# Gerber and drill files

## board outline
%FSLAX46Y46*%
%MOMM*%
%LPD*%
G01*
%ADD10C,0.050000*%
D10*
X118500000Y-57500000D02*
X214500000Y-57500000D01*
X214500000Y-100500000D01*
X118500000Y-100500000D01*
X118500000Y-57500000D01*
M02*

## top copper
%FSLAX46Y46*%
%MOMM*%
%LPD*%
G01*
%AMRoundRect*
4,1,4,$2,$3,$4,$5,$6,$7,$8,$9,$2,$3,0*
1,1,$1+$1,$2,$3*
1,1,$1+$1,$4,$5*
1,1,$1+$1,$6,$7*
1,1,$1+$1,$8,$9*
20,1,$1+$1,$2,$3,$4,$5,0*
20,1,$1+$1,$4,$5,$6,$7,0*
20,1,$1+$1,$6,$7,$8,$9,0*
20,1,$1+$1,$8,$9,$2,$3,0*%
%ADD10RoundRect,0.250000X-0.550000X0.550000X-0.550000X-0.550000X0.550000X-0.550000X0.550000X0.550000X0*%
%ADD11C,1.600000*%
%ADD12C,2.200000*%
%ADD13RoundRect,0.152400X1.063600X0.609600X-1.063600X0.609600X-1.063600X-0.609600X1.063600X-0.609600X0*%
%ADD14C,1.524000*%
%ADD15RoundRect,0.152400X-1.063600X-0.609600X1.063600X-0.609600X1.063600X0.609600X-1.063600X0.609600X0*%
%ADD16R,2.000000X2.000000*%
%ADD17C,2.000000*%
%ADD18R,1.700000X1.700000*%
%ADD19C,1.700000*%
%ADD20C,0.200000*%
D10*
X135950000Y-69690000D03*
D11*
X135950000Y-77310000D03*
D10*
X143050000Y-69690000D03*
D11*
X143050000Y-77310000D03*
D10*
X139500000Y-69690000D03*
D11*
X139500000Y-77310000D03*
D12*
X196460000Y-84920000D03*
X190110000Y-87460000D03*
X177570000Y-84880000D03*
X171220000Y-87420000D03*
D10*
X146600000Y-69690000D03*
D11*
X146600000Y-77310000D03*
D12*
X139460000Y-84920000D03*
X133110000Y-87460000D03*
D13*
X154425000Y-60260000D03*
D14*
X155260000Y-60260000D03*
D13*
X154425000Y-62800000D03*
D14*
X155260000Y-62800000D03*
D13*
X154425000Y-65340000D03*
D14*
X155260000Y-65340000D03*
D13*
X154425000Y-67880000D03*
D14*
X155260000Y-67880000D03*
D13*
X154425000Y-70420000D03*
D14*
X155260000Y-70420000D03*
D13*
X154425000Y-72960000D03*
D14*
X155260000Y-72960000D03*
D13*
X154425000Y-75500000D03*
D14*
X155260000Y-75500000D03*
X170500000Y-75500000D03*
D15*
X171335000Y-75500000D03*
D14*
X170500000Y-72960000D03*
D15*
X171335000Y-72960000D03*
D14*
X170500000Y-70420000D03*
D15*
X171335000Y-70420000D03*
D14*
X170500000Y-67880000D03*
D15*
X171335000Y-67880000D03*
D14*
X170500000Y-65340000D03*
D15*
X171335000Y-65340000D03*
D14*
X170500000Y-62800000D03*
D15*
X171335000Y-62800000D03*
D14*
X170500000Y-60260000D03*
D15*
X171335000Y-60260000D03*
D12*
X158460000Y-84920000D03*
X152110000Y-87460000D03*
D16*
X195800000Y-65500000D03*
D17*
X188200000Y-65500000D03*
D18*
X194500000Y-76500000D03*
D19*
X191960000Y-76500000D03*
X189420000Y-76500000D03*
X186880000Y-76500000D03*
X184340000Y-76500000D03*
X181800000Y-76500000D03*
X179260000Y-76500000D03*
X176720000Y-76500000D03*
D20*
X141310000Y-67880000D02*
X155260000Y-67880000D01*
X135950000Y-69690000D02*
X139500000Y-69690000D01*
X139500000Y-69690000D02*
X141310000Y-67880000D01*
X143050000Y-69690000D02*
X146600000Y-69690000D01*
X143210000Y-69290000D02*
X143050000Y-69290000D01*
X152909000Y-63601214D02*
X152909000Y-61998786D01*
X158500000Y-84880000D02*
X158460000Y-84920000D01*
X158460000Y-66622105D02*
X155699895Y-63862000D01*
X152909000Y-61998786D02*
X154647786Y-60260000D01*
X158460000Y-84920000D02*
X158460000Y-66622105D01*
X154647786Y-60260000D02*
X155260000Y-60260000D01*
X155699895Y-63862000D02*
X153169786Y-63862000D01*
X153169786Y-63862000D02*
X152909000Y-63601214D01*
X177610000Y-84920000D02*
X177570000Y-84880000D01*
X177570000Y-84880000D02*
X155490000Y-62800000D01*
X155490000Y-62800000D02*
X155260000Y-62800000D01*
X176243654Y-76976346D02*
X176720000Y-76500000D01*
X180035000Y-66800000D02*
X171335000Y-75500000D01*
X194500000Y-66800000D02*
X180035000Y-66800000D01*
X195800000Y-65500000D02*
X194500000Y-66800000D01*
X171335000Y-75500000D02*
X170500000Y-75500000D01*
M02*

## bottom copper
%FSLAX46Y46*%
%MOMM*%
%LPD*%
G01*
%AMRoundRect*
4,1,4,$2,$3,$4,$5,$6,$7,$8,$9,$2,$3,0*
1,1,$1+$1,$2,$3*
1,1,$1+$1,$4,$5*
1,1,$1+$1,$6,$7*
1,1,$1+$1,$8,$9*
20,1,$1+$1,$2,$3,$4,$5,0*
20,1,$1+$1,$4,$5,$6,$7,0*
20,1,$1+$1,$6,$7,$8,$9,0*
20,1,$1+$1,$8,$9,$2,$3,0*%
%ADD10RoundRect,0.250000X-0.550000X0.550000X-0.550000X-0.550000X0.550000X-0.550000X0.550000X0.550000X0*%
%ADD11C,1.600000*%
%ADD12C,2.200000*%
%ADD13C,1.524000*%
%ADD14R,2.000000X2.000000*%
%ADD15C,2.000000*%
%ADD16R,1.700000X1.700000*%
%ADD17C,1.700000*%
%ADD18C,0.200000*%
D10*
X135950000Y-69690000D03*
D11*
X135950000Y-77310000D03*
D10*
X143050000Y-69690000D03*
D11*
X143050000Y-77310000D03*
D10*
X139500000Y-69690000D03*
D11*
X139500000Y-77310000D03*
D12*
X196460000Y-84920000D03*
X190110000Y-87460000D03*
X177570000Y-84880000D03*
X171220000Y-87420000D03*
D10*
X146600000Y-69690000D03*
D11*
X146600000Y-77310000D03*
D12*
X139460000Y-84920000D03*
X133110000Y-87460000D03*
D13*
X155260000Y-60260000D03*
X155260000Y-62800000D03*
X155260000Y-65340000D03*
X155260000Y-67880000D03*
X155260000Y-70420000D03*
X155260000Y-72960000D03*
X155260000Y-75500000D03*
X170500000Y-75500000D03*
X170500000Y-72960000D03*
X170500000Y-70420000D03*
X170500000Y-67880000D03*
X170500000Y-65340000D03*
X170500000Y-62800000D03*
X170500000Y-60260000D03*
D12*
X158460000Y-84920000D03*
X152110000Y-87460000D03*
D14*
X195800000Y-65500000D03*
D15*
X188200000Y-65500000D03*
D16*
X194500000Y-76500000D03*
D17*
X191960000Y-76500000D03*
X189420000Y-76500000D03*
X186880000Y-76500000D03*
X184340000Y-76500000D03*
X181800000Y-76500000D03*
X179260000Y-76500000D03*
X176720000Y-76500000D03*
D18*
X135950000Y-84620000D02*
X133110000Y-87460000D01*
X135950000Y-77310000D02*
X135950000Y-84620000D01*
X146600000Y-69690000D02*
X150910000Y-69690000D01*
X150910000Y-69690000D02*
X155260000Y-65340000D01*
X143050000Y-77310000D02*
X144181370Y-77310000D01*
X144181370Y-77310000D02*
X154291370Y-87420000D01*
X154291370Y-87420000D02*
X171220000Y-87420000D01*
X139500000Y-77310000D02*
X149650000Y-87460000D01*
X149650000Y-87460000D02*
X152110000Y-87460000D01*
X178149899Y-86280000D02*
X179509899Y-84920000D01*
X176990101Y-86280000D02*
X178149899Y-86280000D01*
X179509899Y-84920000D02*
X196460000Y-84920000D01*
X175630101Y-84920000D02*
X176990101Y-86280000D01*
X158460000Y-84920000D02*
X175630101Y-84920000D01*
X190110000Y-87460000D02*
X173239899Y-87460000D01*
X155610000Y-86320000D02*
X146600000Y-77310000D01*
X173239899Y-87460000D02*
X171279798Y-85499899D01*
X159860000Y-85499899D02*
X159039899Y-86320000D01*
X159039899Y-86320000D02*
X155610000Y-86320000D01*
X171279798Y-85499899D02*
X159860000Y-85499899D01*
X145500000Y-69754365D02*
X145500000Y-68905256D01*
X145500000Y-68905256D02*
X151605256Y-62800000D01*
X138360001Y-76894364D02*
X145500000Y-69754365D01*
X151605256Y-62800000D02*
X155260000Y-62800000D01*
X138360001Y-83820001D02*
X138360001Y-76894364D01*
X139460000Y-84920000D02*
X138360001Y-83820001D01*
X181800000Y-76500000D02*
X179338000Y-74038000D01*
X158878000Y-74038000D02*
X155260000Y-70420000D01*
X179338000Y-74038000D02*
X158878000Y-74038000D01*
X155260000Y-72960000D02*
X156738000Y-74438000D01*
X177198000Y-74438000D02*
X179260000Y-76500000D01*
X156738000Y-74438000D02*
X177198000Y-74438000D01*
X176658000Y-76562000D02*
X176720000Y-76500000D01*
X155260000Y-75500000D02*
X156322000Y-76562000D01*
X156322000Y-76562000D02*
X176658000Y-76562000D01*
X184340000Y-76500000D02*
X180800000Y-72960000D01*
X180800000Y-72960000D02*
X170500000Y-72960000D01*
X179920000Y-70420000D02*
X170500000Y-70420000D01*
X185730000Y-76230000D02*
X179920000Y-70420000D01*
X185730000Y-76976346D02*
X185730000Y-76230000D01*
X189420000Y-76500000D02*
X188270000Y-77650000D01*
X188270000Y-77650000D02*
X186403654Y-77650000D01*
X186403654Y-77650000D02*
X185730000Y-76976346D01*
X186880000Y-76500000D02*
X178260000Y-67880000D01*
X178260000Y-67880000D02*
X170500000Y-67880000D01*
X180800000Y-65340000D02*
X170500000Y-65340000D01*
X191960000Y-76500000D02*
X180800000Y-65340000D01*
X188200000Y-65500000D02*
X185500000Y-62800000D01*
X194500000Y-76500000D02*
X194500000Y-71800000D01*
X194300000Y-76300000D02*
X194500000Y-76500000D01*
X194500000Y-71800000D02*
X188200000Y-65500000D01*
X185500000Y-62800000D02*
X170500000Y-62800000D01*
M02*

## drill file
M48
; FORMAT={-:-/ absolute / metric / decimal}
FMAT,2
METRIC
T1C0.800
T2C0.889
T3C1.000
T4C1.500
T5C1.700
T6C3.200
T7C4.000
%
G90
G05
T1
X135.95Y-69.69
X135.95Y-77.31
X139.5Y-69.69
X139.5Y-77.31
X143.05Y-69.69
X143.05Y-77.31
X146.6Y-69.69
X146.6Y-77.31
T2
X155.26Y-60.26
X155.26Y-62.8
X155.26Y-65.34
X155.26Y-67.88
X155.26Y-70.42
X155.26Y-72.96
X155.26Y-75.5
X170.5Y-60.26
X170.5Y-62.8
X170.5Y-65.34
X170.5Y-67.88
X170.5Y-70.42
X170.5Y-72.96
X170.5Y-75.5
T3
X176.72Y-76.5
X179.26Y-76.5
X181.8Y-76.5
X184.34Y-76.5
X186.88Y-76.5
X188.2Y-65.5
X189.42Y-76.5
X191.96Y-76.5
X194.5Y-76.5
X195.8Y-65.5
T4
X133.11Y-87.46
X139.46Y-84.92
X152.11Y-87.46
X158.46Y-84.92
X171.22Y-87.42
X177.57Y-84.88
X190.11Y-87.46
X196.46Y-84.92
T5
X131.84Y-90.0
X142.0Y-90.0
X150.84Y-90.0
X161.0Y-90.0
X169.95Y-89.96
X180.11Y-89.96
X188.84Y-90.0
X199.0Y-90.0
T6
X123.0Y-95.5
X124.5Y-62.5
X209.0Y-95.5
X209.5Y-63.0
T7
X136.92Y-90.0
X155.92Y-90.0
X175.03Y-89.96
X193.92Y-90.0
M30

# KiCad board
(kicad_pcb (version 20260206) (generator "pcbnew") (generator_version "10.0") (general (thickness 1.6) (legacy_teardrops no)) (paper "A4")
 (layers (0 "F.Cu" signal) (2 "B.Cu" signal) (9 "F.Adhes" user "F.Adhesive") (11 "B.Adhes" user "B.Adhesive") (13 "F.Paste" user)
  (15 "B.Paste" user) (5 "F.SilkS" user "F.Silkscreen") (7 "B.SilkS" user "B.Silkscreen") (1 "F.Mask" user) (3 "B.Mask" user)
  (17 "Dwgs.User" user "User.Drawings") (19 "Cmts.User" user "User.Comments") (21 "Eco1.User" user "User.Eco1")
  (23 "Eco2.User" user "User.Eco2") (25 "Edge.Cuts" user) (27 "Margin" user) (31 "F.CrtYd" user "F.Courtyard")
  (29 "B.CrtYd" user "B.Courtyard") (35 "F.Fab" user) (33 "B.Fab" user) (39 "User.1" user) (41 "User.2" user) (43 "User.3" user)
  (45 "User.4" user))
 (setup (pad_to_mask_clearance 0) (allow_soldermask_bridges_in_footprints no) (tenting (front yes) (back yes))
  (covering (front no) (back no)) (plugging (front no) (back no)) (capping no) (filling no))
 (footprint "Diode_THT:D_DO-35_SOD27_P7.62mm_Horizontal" (layer "F.Cu") (at 135.95 69.69 -90)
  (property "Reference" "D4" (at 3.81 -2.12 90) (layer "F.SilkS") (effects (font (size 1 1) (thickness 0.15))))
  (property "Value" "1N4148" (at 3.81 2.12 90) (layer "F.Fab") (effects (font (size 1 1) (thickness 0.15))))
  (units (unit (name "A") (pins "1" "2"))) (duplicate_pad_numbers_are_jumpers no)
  (pad "1" thru_hole roundrect (at 0 0 270) (size 1.6 1.6) (drill 0.8) (layers "*.Cu" "*.Mask") (remove_unused_layers no)
   (roundrect_rratio 0.15625) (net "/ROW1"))
  (pad "2" thru_hole circle (at 7.62 0 270) (size 1.6 1.6) (drill 0.8) (layers "*.Cu" "*.Mask") (remove_unused_layers no) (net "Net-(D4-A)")))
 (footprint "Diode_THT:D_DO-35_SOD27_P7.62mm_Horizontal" (layer "F.Cu") (at 143.05 69.69 -90)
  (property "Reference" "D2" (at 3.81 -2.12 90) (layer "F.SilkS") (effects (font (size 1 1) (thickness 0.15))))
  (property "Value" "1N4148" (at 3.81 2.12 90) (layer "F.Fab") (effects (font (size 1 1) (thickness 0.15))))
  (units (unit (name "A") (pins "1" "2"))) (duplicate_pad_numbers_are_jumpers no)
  (pad "1" thru_hole roundrect (at 0 0 270) (size 1.6 1.6) (drill 0.8) (layers "*.Cu" "*.Mask") (remove_unused_layers no)
   (roundrect_rratio 0.15625) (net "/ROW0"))
  (pad "2" thru_hole circle (at 7.62 0 270) (size 1.6 1.6) (drill 0.8) (layers "*.Cu" "*.Mask") (remove_unused_layers no) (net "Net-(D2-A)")))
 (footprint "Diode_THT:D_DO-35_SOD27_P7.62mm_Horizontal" (layer "F.Cu") (at 139.5 69.69 -90)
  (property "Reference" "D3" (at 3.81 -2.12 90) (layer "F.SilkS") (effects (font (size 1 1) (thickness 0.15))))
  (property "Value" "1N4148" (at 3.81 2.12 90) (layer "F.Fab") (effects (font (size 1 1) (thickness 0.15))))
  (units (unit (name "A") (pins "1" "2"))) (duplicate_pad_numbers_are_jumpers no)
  (pad "1" thru_hole roundrect (at 0 0 270) (size 1.6 1.6) (drill 0.8) (layers "*.Cu" "*.Mask") (remove_unused_layers no)
   (roundrect_rratio 0.15625) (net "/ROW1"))
  (pad "2" thru_hole circle (at 7.62 0 270) (size 1.6 1.6) (drill 0.8) (layers "*.Cu" "*.Mask") (remove_unused_layers no) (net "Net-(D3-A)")))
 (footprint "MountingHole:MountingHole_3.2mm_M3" (layer "F.Cu") (at 124.5 62.5)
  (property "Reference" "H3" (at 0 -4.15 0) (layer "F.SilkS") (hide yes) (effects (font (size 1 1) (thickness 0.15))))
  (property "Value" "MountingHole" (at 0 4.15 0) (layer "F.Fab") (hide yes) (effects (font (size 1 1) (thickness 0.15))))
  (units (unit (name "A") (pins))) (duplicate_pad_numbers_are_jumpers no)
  (pad "" np_thru_hole circle (at 0 0) (size 3.2 3.2) (drill 3.2) (layers "*.Cu" "*.Mask")))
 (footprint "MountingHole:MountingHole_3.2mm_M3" (layer "F.Cu") (at 209 95.5)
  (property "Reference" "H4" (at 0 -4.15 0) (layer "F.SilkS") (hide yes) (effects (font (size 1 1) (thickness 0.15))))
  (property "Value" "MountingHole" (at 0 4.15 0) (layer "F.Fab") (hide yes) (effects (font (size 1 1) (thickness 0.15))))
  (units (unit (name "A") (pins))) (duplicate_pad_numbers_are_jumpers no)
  (pad "" np_thru_hole circle (at 0 0) (size 3.2 3.2) (drill 3.2) (layers "*.Cu" "*.Mask")))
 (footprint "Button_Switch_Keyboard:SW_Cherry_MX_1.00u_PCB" (layer "F.Cu") (at 196.46 84.92)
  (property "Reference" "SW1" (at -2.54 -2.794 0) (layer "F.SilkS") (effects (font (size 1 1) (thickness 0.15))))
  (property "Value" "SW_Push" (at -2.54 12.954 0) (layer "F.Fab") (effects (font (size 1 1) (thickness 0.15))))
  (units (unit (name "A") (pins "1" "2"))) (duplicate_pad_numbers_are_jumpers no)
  (pad "" np_thru_hole circle (at -7.62 5.08) (size 1.7 1.7) (drill 1.7) (layers "*.Cu" "*.Mask"))
  (pad "" np_thru_hole circle (at -2.54 5.08) (size 4 4) (drill 4) (layers "*.Cu" "*.Mask"))
  (pad "" np_thru_hole circle (at 2.54 5.08) (size 1.7 1.7) (drill 1.7) (layers "*.Cu" "*.Mask"))
  (pad "1" thru_hole circle (at 0 0) (size 2.2 2.2) (drill 1.5) (layers "*.Cu" "*.Mask") (remove_unused_layers no) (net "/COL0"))
  (pad "2" thru_hole circle (at -6.35 2.54) (size 2.2 2.2) (drill 1.5) (layers "*.Cu" "*.Mask") (remove_unused_layers no) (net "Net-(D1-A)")))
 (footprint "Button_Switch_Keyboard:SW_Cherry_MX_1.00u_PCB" (layer "F.Cu") (at 177.57 84.88)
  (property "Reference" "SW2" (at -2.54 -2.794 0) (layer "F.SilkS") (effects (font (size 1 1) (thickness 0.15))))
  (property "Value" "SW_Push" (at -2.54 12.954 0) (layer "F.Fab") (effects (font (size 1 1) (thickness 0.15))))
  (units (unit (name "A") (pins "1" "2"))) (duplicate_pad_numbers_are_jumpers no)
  (pad "" np_thru_hole circle (at -7.62 5.08) (size 1.7 1.7) (drill 1.7) (layers "*.Cu" "*.Mask"))
  (pad "" np_thru_hole circle (at -2.54 5.08) (size 4 4) (drill 4) (layers "*.Cu" "*.Mask"))
  (pad "" np_thru_hole circle (at 2.54 5.08) (size 1.7 1.7) (drill 1.7) (layers "*.Cu" "*.Mask"))
  (pad "1" thru_hole circle (at 0 0) (size 2.2 2.2) (drill 1.5) (layers "*.Cu" "*.Mask") (remove_unused_layers no) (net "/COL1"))
  (pad "2" thru_hole circle (at -6.35 2.54) (size 2.2 2.2) (drill 1.5) (layers "*.Cu" "*.Mask") (remove_unused_layers no) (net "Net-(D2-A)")))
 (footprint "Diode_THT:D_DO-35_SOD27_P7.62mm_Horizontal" (layer "F.Cu") (at 146.6 69.69 -90)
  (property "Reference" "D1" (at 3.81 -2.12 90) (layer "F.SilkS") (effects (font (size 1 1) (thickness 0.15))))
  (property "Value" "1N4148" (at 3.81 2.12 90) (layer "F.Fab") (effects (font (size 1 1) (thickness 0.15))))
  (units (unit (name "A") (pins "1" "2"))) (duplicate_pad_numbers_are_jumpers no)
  (pad "1" thru_hole roundrect (at 0 0 270) (size 1.6 1.6) (drill 0.8) (layers "*.Cu" "*.Mask") (remove_unused_layers no)
   (roundrect_rratio 0.15625) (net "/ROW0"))
  (pad "2" thru_hole circle (at 7.62 0 270) (size 1.6 1.6) (drill 0.8) (layers "*.Cu" "*.Mask") (remove_unused_layers no) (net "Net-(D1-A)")))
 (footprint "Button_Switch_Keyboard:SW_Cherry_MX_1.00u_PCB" (layer "F.Cu") (at 139.46 84.92)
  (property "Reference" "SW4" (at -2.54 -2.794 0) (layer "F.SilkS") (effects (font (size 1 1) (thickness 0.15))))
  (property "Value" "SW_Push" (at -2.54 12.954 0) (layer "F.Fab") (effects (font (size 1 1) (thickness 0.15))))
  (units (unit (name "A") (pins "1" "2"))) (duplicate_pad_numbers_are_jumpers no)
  (pad "" np_thru_hole circle (at -7.62 5.08) (size 1.7 1.7) (drill 1.7) (layers "*.Cu" "*.Mask"))
  (pad "" np_thru_hole circle (at -2.54 5.08) (size 4 4) (drill 4) (layers "*.Cu" "*.Mask"))
  (pad "" np_thru_hole circle (at 2.54 5.08) (size 1.7 1.7) (drill 1.7) (layers "*.Cu" "*.Mask"))
  (pad "1" thru_hole circle (at 0 0) (size 2.2 2.2) (drill 1.5) (layers "*.Cu" "*.Mask") (remove_unused_layers no) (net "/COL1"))
  (pad "2" thru_hole circle (at -6.35 2.54) (size 2.2 2.2) (drill 1.5) (layers "*.Cu" "*.Mask") (remove_unused_layers no) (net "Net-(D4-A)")))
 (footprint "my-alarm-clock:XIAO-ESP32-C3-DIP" (layer "F.Cu") (at 162.88 67.88 90)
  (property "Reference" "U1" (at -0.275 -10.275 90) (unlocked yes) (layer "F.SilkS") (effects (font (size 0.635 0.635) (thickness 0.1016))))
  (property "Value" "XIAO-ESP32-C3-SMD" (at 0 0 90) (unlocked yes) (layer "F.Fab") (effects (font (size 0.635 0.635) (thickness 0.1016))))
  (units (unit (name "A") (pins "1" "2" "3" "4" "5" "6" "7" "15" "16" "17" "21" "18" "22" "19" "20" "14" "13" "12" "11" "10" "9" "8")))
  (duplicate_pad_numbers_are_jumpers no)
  (pad "1" smd roundrect (at 7.62 -8.455 180) (size 2.432 1.524) (layers "F.Cu" "F.Mask") (roundrect_rratio 0.1) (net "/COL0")
   (thermal_bridge_angle 45))
  (pad "1" thru_hole circle (at 7.62 -7.62 180) (size 1.524 1.524) (drill 0.889) (layers "*.Cu" "*.Mask") (remove_unused_layers no)
   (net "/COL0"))
  (pad "2" smd roundrect (at 5.08 -8.455 180) (size 2.432 1.524) (layers "F.Cu" "F.Mask") (roundrect_rratio 0.1) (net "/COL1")
   (thermal_bridge_angle 45))
  (pad "2" thru_hole circle (at 5.08 -7.62 180) (size 1.524 1.524) (drill 0.889) (layers "*.Cu" "*.Mask") (remove_unused_layers no)
   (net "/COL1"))
  (pad "3" smd roundrect (at 2.54 -8.455 180) (size 2.432 1.524) (layers "F.Cu" "F.Mask") (roundrect_rratio 0.1) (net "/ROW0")
   (thermal_bridge_angle 45))
  (pad "3" thru_hole circle (at 2.54 -7.62 180) (size 1.524 1.524) (drill 0.889) (layers "*.Cu" "*.Mask") (remove_unused_layers no)
   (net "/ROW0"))
  (pad "4" smd roundrect (at 0 -8.455 180) (size 2.432 1.524) (layers "F.Cu" "F.Mask") (roundrect_rratio 0.1) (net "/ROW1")
   (thermal_bridge_angle 45))
  (pad "4" thru_hole circle (at 0 -7.62 180) (size 1.524 1.524) (drill 0.889) (layers "*.Cu" "*.Mask") (remove_unused_layers no)
   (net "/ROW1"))
  (pad "5" smd roundrect (at -2.54 -8.455 180) (size 2.432 1.524) (layers "F.Cu" "F.Mask") (roundrect_rratio 0.1) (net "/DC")
   (thermal_bridge_angle 45))
  (pad "5" thru_hole circle (at -2.54 -7.62 180) (size 1.524 1.524) (drill 0.889) (layers "*.Cu" "*.Mask") (remove_unused_layers no)
   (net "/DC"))
  (pad "6" smd roundrect (at -5.08 -8.455 180) (size 2.432 1.524) (layers "F.Cu" "F.Mask") (roundrect_rratio 0.1) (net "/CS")
   (thermal_bridge_angle 45))
  (pad "6" thru_hole circle (at -5.08 -7.62 180) (size 1.524 1.524) (drill 0.889) (layers "*.Cu" "*.Mask") (remove_unused_layers no)
   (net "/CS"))
  (pad "7" smd roundrect (at -7.62 -8.455 180) (size 2.432 1.524) (layers "F.Cu" "F.Mask") (roundrect_rratio 0.1) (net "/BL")
   (thermal_bridge_angle 45))
  (pad "7" thru_hole circle (at -7.62 -7.62 180) (size 1.524 1.524) (drill 0.889) (layers "*.Cu" "*.Mask") (remove_unused_layers no)
   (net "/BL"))
  (pad "8" thru_hole circle (at -7.62 7.62) (size 1.524 1.524) (drill 0.889) (layers "*.Cu" "*.Mask") (remove_unused_layers no)
   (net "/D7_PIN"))
  (pad "8" smd roundrect (at -7.62 8.455) (size 2.432 1.524) (layers "F.Cu" "F.Mask") (roundrect_rratio 0.1) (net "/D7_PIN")
   (thermal_bridge_angle 45))
  (pad "9" thru_hole circle (at -5.08 7.62) (size 1.524 1.524) (drill 0.889) (layers "*.Cu" "*.Mask") (remove_unused_layers no) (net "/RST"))
  (pad "9" smd roundrect (at -5.08 8.455) (size 2.432 1.524) (layers "F.Cu" "F.Mask") (roundrect_rratio 0.1) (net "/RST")
   (thermal_bridge_angle 45))
  (pad "10" thru_hole circle (at -2.54 7.62) (size 1.524 1.524) (drill 0.889) (layers "*.Cu" "*.Mask") (remove_unused_layers no)
   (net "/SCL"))
  (pad "10" smd roundrect (at -2.54 8.455) (size 2.432 1.524) (layers "F.Cu" "F.Mask") (roundrect_rratio 0.1) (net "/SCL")
   (thermal_bridge_angle 45))
  (pad "11" thru_hole circle (at 0 7.62) (size 1.524 1.524) (drill 0.889) (layers "*.Cu" "*.Mask") (remove_unused_layers no) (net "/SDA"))
  (pad "11" smd roundrect (at 0 8.455) (size 2.432 1.524) (layers "F.Cu" "F.Mask") (roundrect_rratio 0.1) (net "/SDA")
   (thermal_bridge_angle 45))
  (pad "12" thru_hole circle (at 2.54 7.62) (size 1.524 1.524) (drill 0.889) (layers "*.Cu" "*.Mask") (remove_unused_layers no)
   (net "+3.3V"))
  (pad "12" smd roundrect (at 2.54 8.455) (size 2.432 1.524) (layers "F.Cu" "F.Mask") (roundrect_rratio 0.1) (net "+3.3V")
   (thermal_bridge_angle 45))
  (pad "13" thru_hole circle (at 5.08 7.62) (size 1.524 1.524) (drill 0.889) (layers "*.Cu" "*.Mask") (remove_unused_layers no) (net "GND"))
  (pad "13" smd roundrect (at 5.08 8.455) (size 2.432 1.524) (layers "F.Cu" "F.Mask") (roundrect_rratio 0.1) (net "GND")
   (thermal_bridge_angle 45))
  (pad "14" thru_hole circle (at 7.62 7.62) (size 1.524 1.524) (drill 0.889) (layers "*.Cu" "*.Mask") (remove_unused_layers no)
   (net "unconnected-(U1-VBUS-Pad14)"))
  (pad "14" smd roundrect (at 7.62 8.455) (size 2.432 1.524) (layers "F.Cu" "F.Mask") (roundrect_rratio 0.1)
   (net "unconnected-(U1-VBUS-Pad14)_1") (thermal_bridge_angle 45)))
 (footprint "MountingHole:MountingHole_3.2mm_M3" (layer "F.Cu") (at 209.5 63)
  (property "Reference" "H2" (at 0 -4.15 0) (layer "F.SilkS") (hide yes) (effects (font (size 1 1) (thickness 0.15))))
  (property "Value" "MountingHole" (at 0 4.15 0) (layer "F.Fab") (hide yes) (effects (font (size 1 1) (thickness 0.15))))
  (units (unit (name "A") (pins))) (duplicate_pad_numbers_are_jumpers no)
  (pad "" np_thru_hole circle (at 0 0) (size 3.2 3.2) (drill 3.2) (layers "*.Cu" "*.Mask")))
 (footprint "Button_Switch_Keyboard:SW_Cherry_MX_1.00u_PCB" (layer "F.Cu") (at 158.46 84.92)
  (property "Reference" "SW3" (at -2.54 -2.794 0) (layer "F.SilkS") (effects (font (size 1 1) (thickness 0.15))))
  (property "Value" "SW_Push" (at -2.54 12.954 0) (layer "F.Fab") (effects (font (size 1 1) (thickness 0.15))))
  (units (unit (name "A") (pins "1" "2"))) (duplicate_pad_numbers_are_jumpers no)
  (pad "" np_thru_hole circle (at -7.62 5.08) (size 1.7 1.7) (drill 1.7) (layers "*.Cu" "*.Mask"))
  (pad "" np_thru_hole circle (at -2.54 5.08) (size 4 4) (drill 4) (layers "*.Cu" "*.Mask"))
  (pad "" np_thru_hole circle (at 2.54 5.08) (size 1.7 1.7) (drill 1.7) (layers "*.Cu" "*.Mask"))
  (pad "1" thru_hole circle (at 0 0) (size 2.2 2.2) (drill 1.5) (layers "*.Cu" "*.Mask") (remove_unused_layers no) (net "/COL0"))
  (pad "2" thru_hole circle (at -6.35 2.54) (size 2.2 2.2) (drill 1.5) (layers "*.Cu" "*.Mask") (remove_unused_layers no) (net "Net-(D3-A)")))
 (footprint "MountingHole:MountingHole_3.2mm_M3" (layer "F.Cu") (at 123 95.5)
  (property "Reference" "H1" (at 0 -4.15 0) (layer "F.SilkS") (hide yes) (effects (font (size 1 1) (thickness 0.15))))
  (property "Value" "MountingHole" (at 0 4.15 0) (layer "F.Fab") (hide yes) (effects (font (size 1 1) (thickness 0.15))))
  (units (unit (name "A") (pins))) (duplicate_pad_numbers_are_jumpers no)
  (pad "" np_thru_hole circle (at 0 0) (size 3.2 3.2) (drill 3.2) (layers "*.Cu" "*.Mask")))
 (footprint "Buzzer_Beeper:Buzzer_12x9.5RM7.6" (layer "B.Cu") (at 195.8 65.5 180)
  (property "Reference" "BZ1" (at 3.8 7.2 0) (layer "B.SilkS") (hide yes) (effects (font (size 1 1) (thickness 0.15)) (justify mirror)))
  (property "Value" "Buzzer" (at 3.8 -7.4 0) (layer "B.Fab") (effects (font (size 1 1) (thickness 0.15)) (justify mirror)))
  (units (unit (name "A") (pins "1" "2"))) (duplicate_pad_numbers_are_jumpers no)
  (pad "1" thru_hole rect (at 0 0 180) (size 2 2) (drill 1) (layers "*.Cu" "*.Mask") (remove_unused_layers no) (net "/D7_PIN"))
  (pad "2" thru_hole circle (at 7.6 0 180) (size 2 2) (drill 1) (layers "*.Cu" "*.Mask") (remove_unused_layers no) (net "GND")))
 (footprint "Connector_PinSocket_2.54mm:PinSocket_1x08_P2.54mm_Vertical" (layer "B.Cu") (at 194.5 76.5 90)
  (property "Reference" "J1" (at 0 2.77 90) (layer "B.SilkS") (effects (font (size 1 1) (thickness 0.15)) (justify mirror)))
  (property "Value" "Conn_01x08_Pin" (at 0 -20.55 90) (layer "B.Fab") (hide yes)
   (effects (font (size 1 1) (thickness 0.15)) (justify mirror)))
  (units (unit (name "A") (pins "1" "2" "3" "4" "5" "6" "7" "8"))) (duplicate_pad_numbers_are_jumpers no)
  (pad "1" thru_hole rect (at 0 0 90) (size 1.7 1.7) (drill 1) (layers "*.Cu" "*.Mask") (remove_unused_layers no) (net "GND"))
  (pad "2" thru_hole circle (at 0 -2.54 90) (size 1.7 1.7) (drill 1) (layers "*.Cu" "*.Mask") (remove_unused_layers no) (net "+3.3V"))
  (pad "3" thru_hole circle (at 0 -5.08 90) (size 1.7 1.7) (drill 1) (layers "*.Cu" "*.Mask") (remove_unused_layers no) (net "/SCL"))
  (pad "4" thru_hole circle (at 0 -7.62 90) (size 1.7 1.7) (drill 1) (layers "*.Cu" "*.Mask") (remove_unused_layers no) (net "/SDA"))
  (pad "5" thru_hole circle (at 0 -10.16 90) (size 1.7 1.7) (drill 1) (layers "*.Cu" "*.Mask") (remove_unused_layers no) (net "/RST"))
  (pad "6" thru_hole circle (at 0 -12.7 90) (size 1.7 1.7) (drill 1) (layers "*.Cu" "*.Mask") (remove_unused_layers no) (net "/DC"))
  (pad "7" thru_hole circle (at 0 -15.24 90) (size 1.7 1.7) (drill 1) (layers "*.Cu" "*.Mask") (remove_unused_layers no) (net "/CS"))
  (pad "8" thru_hole circle (at 0 -17.78 90) (size 1.7 1.7) (drill 1) (layers "*.Cu" "*.Mask") (remove_unused_layers no) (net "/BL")))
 (gr_rect (start 118.5 57.5) (end 214.5 100.5) (stroke (width 0.05) (type default)) (fill no) (layer "Edge.Cuts"))
 (segment (start 141.31 67.88) (end 155.26 67.88) (width 0.2) (layer "F.Cu") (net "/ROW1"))
 (segment (start 135.95 69.69) (end 139.5 69.69) (width 0.2) (layer "F.Cu") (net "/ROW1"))
 (segment (start 139.5 69.69) (end 141.31 67.88) (width 0.2) (layer "F.Cu") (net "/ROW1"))
 (segment (start 135.95 84.62) (end 133.11 87.46) (width 0.2) (layer "B.Cu") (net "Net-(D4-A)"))
 (segment (start 135.95 77.31) (end 135.95 84.62) (width 0.2) (layer "B.Cu") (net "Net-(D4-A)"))
 (segment (start 143.05 69.69) (end 146.6 69.69) (width 0.2) (layer "F.Cu") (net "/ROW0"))
 (segment (start 143.21 69.29) (end 143.05 69.29) (width 0.2) (layer "F.Cu") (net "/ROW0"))
 (segment (start 146.6 69.69) (end 150.91 69.69) (width 0.2) (layer "B.Cu") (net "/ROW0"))
 (segment (start 150.91 69.69) (end 155.26 65.34) (width 0.2) (layer "B.Cu") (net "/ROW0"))
 (segment (start 143.05 77.31) (end 144.18137 77.31) (width 0.2) (layer "B.Cu") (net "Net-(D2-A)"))
 (segment (start 144.18137 77.31) (end 154.29137 87.42) (width 0.2) (layer "B.Cu") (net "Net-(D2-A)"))
 (segment (start 154.29137 87.42) (end 171.22 87.42) (width 0.2) (layer "B.Cu") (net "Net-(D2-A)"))
 (segment (start 139.5 77.31) (end 149.65 87.46) (width 0.2) (layer "B.Cu") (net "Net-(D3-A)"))
 (segment (start 149.65 87.46) (end 152.11 87.46) (width 0.2) (layer "B.Cu") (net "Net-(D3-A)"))
 (segment (start 152.909 63.601214) (end 152.909 61.998786) (width 0.2) (layer "F.Cu") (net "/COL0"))
 (segment (start 158.5 84.88) (end 158.46 84.92) (width 0.2) (layer "F.Cu") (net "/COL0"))
 (segment (start 158.46 66.622105) (end 155.699895 63.862) (width 0.2) (layer "F.Cu") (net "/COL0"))
 (segment (start 152.909 61.998786) (end 154.647786 60.26) (width 0.2) (layer "F.Cu") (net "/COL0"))
 (segment (start 158.46 84.92) (end 158.46 66.622105) (width 0.2) (layer "F.Cu") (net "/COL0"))
 (segment (start 154.647786 60.26) (end 155.26 60.26) (width 0.2) (layer "F.Cu") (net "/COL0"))
 (segment (start 155.699895 63.862) (end 153.169786 63.862) (width 0.2) (layer "F.Cu") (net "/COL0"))
 (segment (start 153.169786 63.862) (end 152.909 63.601214) (width 0.2) (layer "F.Cu") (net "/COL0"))
 (segment (start 178.149899 86.28) (end 179.509899 84.92) (width 0.2) (layer "B.Cu") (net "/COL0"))
 (segment (start 176.990101 86.28) (end 178.149899 86.28) (width 0.2) (layer "B.Cu") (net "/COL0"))
 (segment (start 179.509899 84.92) (end 196.46 84.92) (width 0.2) (layer "B.Cu") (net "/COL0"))
 (segment (start 175.630101 84.92) (end 176.990101 86.28) (width 0.2) (layer "B.Cu") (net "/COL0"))
 (segment (start 158.46 84.92) (end 175.630101 84.92) (width 0.2) (layer "B.Cu") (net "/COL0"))
 (segment (start 190.11 87.46) (end 173.239899 87.46) (width 0.2) (layer "B.Cu") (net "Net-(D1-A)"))
 (segment (start 155.61 86.32) (end 146.6 77.31) (width 0.2) (layer "B.Cu") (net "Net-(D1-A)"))
 (segment (start 173.239899 87.46) (end 171.279798 85.499899) (width 0.2) (layer "B.Cu") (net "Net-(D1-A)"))
 (segment (start 159.86 85.499899) (end 159.039899 86.32) (width 0.2) (layer "B.Cu") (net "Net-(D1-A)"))
 (segment (start 159.039899 86.32) (end 155.61 86.32) (width 0.2) (layer "B.Cu") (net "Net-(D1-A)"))
 (segment (start 171.279798 85.499899) (end 159.86 85.499899) (width 0.2) (layer "B.Cu") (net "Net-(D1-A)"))
 (segment (start 177.61 84.92) (end 177.57 84.88) (width 0.2) (layer "F.Cu") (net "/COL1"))
 (segment (start 177.57 84.88) (end 155.49 62.8) (width 0.2) (layer "F.Cu") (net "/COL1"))
 (segment (start 155.49 62.8) (end 155.26 62.8) (width 0.2) (layer "F.Cu") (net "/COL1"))
 (segment (start 145.5 69.754365) (end 145.5 68.905256) (width 0.2) (layer "B.Cu") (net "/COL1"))
 (segment (start 145.5 68.905256) (end 151.605256 62.8) (width 0.2) (layer "B.Cu") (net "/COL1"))
 (segment (start 138.360001 76.894364) (end 145.5 69.754365) (width 0.2) (layer "B.Cu") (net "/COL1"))
 (segment (start 151.605256 62.8) (end 155.26 62.8) (width 0.2) (layer "B.Cu") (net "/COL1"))
 (segment (start 138.360001 83.820001) (end 138.360001 76.894364) (width 0.2) (layer "B.Cu") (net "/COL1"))
 (segment (start 139.46 84.92) (end 138.360001 83.820001) (width 0.2) (layer "B.Cu") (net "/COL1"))
 (segment (start 181.8 76.5) (end 179.338 74.038) (width 0.2) (layer "B.Cu") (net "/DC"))
 (segment (start 158.878 74.038) (end 155.26 70.42) (width 0.2) (layer "B.Cu") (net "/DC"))
 (segment (start 179.338 74.038) (end 158.878 74.038) (width 0.2) (layer "B.Cu") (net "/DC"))
 (segment (start 155.26 72.96) (end 156.738 74.438) (width 0.2) (layer "B.Cu") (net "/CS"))
 (segment (start 177.198 74.438) (end 179.26 76.5) (width 0.2) (layer "B.Cu") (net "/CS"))
 (segment (start 156.738 74.438) (end 177.198 74.438) (width 0.2) (layer "B.Cu") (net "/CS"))
 (segment (start 176.243654 76.976346) (end 176.72 76.5) (width 0.2) (layer "F.Cu") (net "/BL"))
 (segment (start 176.658 76.562) (end 176.72 76.5) (width 0.2) (layer "B.Cu") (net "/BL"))
 (segment (start 155.26 75.5) (end 156.322 76.562) (width 0.2) (layer "B.Cu") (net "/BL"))
 (segment (start 156.322 76.562) (end 176.658 76.562) (width 0.2) (layer "B.Cu") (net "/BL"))
 (segment (start 180.035 66.8) (end 171.335 75.5) (width 0.2) (layer "F.Cu") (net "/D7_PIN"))
 (segment (start 194.5 66.8) (end 180.035 66.8) (width 0.2) (layer "F.Cu") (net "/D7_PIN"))
 (segment (start 195.8 65.5) (end 194.5 66.8) (width 0.2) (layer "F.Cu") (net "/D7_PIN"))
 (segment (start 171.335 75.5) (end 170.5 75.5) (width 0.2) (layer "F.Cu") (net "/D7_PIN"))
 (segment (start 184.34 76.5) (end 180.8 72.96) (width 0.2) (layer "B.Cu") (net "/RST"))
 (segment (start 180.8 72.96) (end 170.5 72.96) (width 0.2) (layer "B.Cu") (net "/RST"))
 (segment (start 179.92 70.42) (end 170.5 70.42) (width 0.2) (layer "B.Cu") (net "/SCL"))
 (segment (start 185.73 76.23) (end 179.92 70.42) (width 0.2) (layer "B.Cu") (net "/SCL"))
 (segment (start 185.73 76.976346) (end 185.73 76.23) (width 0.2) (layer "B.Cu") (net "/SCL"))
 (segment (start 189.42 76.5) (end 188.27 77.65) (width 0.2) (layer "B.Cu") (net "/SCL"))
 (segment (start 188.27 77.65) (end 186.403654 77.65) (width 0.2) (layer "B.Cu") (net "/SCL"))
 (segment (start 186.403654 77.65) (end 185.73 76.976346) (width 0.2) (layer "B.Cu") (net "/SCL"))
 (segment (start 186.88 76.5) (end 178.26 67.88) (width 0.2) (layer "B.Cu") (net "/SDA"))
 (segment (start 178.26 67.88) (end 170.5 67.88) (width 0.2) (layer "B.Cu") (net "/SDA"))
 (segment (start 180.8 65.34) (end 170.5 65.34) (width 0.2) (layer "B.Cu") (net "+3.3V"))
 (segment (start 191.96 76.5) (end 180.8 65.34) (width 0.2) (layer "B.Cu") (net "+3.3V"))
 (segment (start 188.2 65.5) (end 185.5 62.8) (width 0.2) (layer "B.Cu") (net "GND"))
 (segment (start 194.5 76.5) (end 194.5 71.8) (width 0.2) (layer "B.Cu") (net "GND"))
 (segment (start 194.3 76.3) (end 194.5 76.5) (width 0.2) (layer "B.Cu") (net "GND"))
 (segment (start 194.5 71.8) (end 188.2 65.5) (width 0.2) (layer "B.Cu") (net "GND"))
 (segment (start 185.5 62.8) (end 170.5 62.8) (width 0.2) (layer "B.Cu") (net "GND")))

